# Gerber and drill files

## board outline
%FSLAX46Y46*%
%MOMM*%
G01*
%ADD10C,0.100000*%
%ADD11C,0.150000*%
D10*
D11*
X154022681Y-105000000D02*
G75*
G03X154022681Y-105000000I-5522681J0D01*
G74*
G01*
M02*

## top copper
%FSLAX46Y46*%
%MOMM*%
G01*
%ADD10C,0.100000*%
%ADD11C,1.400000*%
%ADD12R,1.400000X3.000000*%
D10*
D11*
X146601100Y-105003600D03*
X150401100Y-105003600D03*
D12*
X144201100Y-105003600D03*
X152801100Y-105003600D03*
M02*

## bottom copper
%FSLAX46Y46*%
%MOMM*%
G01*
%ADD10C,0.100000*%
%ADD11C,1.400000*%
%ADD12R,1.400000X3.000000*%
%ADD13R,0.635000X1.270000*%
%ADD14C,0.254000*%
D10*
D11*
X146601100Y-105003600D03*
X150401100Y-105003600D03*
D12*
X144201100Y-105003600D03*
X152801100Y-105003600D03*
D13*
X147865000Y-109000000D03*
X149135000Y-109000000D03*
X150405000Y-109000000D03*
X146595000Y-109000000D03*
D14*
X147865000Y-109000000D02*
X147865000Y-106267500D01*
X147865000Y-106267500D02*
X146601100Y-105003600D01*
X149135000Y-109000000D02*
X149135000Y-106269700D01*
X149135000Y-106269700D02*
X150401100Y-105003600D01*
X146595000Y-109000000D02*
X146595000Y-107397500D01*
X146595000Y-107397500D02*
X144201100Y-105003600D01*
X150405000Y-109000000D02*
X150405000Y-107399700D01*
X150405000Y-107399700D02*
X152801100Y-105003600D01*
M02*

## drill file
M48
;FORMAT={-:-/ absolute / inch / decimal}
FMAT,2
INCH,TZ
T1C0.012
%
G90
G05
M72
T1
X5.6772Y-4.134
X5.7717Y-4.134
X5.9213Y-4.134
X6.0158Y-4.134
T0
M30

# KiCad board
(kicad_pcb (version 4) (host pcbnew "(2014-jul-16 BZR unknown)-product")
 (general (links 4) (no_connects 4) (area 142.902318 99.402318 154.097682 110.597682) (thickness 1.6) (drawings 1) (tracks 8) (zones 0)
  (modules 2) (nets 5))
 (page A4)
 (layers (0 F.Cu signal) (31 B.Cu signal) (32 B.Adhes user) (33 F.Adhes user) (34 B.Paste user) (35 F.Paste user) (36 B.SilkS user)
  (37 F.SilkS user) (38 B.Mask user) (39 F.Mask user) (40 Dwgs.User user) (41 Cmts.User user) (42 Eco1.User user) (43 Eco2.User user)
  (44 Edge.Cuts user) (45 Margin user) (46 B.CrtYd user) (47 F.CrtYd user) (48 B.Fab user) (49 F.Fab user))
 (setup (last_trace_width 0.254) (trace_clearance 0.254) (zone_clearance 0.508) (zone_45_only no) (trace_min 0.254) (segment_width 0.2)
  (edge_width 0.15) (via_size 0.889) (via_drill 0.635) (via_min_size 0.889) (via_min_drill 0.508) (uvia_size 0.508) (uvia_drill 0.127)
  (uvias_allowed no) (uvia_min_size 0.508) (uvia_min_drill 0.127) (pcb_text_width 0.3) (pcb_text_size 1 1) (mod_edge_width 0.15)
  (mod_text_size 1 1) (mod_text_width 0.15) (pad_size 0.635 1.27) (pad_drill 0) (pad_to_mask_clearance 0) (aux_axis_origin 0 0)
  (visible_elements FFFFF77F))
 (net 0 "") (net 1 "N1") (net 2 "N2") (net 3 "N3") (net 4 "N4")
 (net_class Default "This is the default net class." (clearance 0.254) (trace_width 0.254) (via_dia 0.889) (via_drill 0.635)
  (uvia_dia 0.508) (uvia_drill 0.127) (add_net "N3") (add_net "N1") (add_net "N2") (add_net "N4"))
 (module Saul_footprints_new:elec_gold (layer F.Cu) (at 148.5011 105.0036)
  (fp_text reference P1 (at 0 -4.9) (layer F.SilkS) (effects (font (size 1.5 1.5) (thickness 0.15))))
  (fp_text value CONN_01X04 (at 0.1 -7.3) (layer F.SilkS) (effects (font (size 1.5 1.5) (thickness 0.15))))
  (pad 2 thru_hole circle (at -1.9 0) (size 1.4 1.4) (drill 0.3) (layers *.Cu *.Mask F.SilkS) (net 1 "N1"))
  (pad 3 thru_hole circle (at 1.9 0) (size 1.4 1.4) (drill 0.3) (layers *.Cu *.Mask F.SilkS) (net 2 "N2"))
  (pad 1 thru_hole rect (at -4.3 0) (size 1.4 3) (drill 0.3) (layers *.Cu *.Mask F.SilkS) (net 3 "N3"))
  (pad 4 thru_hole rect (at 4.3 0) (size 1.4 3) (drill 0.3) (layers *.Cu *.Mask F.SilkS) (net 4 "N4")))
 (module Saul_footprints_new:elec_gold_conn (layer F.Cu) (at 148.5 109)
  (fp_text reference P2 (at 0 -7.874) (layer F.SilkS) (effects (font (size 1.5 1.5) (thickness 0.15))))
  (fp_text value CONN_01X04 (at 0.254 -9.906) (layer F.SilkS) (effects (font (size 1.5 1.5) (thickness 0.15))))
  (pad 2 smd rect (at -0.635 0) (size 0.635 1.27) (layers B.Cu B.Mask) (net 1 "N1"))
  (pad 3 smd rect (at 0.635 0) (size 0.635 1.27) (layers B.Cu B.Mask) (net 2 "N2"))
  (pad 4 smd rect (at 1.905 0) (size 0.635 1.27) (layers B.Cu B.Mask) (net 4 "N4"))
  (pad 1 smd rect (at -1.905 0) (size 0.635 1.27) (layers B.Cu B.Mask) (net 3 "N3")))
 (gr_circle (center 148.5 105) (end 154 104.5) (layer Edge.Cuts) (width 0.15))
 (segment (start 147.865 109) (end 147.865 106.2675) (width 0.254) (layer B.Cu) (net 1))
 (segment (start 147.865 106.2675) (end 146.6011 105.0036) (width 0.254) (layer B.Cu) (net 1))
 (segment (start 149.135 109) (end 149.135 106.2697) (width 0.254) (layer B.Cu) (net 2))
 (segment (start 149.135 106.2697) (end 150.4011 105.0036) (width 0.254) (layer B.Cu) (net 2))
 (segment (start 146.595 109) (end 146.595 107.3975) (width 0.254) (layer B.Cu) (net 3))
 (segment (start 146.595 107.3975) (end 144.2011 105.0036) (width 0.254) (layer B.Cu) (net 3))
 (segment (start 150.405 109) (end 150.405 107.3997) (width 0.254) (layer B.Cu) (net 4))
 (segment (start 150.405 107.3997) (end 152.8011 105.0036) (width 0.254) (layer B.Cu) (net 4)))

